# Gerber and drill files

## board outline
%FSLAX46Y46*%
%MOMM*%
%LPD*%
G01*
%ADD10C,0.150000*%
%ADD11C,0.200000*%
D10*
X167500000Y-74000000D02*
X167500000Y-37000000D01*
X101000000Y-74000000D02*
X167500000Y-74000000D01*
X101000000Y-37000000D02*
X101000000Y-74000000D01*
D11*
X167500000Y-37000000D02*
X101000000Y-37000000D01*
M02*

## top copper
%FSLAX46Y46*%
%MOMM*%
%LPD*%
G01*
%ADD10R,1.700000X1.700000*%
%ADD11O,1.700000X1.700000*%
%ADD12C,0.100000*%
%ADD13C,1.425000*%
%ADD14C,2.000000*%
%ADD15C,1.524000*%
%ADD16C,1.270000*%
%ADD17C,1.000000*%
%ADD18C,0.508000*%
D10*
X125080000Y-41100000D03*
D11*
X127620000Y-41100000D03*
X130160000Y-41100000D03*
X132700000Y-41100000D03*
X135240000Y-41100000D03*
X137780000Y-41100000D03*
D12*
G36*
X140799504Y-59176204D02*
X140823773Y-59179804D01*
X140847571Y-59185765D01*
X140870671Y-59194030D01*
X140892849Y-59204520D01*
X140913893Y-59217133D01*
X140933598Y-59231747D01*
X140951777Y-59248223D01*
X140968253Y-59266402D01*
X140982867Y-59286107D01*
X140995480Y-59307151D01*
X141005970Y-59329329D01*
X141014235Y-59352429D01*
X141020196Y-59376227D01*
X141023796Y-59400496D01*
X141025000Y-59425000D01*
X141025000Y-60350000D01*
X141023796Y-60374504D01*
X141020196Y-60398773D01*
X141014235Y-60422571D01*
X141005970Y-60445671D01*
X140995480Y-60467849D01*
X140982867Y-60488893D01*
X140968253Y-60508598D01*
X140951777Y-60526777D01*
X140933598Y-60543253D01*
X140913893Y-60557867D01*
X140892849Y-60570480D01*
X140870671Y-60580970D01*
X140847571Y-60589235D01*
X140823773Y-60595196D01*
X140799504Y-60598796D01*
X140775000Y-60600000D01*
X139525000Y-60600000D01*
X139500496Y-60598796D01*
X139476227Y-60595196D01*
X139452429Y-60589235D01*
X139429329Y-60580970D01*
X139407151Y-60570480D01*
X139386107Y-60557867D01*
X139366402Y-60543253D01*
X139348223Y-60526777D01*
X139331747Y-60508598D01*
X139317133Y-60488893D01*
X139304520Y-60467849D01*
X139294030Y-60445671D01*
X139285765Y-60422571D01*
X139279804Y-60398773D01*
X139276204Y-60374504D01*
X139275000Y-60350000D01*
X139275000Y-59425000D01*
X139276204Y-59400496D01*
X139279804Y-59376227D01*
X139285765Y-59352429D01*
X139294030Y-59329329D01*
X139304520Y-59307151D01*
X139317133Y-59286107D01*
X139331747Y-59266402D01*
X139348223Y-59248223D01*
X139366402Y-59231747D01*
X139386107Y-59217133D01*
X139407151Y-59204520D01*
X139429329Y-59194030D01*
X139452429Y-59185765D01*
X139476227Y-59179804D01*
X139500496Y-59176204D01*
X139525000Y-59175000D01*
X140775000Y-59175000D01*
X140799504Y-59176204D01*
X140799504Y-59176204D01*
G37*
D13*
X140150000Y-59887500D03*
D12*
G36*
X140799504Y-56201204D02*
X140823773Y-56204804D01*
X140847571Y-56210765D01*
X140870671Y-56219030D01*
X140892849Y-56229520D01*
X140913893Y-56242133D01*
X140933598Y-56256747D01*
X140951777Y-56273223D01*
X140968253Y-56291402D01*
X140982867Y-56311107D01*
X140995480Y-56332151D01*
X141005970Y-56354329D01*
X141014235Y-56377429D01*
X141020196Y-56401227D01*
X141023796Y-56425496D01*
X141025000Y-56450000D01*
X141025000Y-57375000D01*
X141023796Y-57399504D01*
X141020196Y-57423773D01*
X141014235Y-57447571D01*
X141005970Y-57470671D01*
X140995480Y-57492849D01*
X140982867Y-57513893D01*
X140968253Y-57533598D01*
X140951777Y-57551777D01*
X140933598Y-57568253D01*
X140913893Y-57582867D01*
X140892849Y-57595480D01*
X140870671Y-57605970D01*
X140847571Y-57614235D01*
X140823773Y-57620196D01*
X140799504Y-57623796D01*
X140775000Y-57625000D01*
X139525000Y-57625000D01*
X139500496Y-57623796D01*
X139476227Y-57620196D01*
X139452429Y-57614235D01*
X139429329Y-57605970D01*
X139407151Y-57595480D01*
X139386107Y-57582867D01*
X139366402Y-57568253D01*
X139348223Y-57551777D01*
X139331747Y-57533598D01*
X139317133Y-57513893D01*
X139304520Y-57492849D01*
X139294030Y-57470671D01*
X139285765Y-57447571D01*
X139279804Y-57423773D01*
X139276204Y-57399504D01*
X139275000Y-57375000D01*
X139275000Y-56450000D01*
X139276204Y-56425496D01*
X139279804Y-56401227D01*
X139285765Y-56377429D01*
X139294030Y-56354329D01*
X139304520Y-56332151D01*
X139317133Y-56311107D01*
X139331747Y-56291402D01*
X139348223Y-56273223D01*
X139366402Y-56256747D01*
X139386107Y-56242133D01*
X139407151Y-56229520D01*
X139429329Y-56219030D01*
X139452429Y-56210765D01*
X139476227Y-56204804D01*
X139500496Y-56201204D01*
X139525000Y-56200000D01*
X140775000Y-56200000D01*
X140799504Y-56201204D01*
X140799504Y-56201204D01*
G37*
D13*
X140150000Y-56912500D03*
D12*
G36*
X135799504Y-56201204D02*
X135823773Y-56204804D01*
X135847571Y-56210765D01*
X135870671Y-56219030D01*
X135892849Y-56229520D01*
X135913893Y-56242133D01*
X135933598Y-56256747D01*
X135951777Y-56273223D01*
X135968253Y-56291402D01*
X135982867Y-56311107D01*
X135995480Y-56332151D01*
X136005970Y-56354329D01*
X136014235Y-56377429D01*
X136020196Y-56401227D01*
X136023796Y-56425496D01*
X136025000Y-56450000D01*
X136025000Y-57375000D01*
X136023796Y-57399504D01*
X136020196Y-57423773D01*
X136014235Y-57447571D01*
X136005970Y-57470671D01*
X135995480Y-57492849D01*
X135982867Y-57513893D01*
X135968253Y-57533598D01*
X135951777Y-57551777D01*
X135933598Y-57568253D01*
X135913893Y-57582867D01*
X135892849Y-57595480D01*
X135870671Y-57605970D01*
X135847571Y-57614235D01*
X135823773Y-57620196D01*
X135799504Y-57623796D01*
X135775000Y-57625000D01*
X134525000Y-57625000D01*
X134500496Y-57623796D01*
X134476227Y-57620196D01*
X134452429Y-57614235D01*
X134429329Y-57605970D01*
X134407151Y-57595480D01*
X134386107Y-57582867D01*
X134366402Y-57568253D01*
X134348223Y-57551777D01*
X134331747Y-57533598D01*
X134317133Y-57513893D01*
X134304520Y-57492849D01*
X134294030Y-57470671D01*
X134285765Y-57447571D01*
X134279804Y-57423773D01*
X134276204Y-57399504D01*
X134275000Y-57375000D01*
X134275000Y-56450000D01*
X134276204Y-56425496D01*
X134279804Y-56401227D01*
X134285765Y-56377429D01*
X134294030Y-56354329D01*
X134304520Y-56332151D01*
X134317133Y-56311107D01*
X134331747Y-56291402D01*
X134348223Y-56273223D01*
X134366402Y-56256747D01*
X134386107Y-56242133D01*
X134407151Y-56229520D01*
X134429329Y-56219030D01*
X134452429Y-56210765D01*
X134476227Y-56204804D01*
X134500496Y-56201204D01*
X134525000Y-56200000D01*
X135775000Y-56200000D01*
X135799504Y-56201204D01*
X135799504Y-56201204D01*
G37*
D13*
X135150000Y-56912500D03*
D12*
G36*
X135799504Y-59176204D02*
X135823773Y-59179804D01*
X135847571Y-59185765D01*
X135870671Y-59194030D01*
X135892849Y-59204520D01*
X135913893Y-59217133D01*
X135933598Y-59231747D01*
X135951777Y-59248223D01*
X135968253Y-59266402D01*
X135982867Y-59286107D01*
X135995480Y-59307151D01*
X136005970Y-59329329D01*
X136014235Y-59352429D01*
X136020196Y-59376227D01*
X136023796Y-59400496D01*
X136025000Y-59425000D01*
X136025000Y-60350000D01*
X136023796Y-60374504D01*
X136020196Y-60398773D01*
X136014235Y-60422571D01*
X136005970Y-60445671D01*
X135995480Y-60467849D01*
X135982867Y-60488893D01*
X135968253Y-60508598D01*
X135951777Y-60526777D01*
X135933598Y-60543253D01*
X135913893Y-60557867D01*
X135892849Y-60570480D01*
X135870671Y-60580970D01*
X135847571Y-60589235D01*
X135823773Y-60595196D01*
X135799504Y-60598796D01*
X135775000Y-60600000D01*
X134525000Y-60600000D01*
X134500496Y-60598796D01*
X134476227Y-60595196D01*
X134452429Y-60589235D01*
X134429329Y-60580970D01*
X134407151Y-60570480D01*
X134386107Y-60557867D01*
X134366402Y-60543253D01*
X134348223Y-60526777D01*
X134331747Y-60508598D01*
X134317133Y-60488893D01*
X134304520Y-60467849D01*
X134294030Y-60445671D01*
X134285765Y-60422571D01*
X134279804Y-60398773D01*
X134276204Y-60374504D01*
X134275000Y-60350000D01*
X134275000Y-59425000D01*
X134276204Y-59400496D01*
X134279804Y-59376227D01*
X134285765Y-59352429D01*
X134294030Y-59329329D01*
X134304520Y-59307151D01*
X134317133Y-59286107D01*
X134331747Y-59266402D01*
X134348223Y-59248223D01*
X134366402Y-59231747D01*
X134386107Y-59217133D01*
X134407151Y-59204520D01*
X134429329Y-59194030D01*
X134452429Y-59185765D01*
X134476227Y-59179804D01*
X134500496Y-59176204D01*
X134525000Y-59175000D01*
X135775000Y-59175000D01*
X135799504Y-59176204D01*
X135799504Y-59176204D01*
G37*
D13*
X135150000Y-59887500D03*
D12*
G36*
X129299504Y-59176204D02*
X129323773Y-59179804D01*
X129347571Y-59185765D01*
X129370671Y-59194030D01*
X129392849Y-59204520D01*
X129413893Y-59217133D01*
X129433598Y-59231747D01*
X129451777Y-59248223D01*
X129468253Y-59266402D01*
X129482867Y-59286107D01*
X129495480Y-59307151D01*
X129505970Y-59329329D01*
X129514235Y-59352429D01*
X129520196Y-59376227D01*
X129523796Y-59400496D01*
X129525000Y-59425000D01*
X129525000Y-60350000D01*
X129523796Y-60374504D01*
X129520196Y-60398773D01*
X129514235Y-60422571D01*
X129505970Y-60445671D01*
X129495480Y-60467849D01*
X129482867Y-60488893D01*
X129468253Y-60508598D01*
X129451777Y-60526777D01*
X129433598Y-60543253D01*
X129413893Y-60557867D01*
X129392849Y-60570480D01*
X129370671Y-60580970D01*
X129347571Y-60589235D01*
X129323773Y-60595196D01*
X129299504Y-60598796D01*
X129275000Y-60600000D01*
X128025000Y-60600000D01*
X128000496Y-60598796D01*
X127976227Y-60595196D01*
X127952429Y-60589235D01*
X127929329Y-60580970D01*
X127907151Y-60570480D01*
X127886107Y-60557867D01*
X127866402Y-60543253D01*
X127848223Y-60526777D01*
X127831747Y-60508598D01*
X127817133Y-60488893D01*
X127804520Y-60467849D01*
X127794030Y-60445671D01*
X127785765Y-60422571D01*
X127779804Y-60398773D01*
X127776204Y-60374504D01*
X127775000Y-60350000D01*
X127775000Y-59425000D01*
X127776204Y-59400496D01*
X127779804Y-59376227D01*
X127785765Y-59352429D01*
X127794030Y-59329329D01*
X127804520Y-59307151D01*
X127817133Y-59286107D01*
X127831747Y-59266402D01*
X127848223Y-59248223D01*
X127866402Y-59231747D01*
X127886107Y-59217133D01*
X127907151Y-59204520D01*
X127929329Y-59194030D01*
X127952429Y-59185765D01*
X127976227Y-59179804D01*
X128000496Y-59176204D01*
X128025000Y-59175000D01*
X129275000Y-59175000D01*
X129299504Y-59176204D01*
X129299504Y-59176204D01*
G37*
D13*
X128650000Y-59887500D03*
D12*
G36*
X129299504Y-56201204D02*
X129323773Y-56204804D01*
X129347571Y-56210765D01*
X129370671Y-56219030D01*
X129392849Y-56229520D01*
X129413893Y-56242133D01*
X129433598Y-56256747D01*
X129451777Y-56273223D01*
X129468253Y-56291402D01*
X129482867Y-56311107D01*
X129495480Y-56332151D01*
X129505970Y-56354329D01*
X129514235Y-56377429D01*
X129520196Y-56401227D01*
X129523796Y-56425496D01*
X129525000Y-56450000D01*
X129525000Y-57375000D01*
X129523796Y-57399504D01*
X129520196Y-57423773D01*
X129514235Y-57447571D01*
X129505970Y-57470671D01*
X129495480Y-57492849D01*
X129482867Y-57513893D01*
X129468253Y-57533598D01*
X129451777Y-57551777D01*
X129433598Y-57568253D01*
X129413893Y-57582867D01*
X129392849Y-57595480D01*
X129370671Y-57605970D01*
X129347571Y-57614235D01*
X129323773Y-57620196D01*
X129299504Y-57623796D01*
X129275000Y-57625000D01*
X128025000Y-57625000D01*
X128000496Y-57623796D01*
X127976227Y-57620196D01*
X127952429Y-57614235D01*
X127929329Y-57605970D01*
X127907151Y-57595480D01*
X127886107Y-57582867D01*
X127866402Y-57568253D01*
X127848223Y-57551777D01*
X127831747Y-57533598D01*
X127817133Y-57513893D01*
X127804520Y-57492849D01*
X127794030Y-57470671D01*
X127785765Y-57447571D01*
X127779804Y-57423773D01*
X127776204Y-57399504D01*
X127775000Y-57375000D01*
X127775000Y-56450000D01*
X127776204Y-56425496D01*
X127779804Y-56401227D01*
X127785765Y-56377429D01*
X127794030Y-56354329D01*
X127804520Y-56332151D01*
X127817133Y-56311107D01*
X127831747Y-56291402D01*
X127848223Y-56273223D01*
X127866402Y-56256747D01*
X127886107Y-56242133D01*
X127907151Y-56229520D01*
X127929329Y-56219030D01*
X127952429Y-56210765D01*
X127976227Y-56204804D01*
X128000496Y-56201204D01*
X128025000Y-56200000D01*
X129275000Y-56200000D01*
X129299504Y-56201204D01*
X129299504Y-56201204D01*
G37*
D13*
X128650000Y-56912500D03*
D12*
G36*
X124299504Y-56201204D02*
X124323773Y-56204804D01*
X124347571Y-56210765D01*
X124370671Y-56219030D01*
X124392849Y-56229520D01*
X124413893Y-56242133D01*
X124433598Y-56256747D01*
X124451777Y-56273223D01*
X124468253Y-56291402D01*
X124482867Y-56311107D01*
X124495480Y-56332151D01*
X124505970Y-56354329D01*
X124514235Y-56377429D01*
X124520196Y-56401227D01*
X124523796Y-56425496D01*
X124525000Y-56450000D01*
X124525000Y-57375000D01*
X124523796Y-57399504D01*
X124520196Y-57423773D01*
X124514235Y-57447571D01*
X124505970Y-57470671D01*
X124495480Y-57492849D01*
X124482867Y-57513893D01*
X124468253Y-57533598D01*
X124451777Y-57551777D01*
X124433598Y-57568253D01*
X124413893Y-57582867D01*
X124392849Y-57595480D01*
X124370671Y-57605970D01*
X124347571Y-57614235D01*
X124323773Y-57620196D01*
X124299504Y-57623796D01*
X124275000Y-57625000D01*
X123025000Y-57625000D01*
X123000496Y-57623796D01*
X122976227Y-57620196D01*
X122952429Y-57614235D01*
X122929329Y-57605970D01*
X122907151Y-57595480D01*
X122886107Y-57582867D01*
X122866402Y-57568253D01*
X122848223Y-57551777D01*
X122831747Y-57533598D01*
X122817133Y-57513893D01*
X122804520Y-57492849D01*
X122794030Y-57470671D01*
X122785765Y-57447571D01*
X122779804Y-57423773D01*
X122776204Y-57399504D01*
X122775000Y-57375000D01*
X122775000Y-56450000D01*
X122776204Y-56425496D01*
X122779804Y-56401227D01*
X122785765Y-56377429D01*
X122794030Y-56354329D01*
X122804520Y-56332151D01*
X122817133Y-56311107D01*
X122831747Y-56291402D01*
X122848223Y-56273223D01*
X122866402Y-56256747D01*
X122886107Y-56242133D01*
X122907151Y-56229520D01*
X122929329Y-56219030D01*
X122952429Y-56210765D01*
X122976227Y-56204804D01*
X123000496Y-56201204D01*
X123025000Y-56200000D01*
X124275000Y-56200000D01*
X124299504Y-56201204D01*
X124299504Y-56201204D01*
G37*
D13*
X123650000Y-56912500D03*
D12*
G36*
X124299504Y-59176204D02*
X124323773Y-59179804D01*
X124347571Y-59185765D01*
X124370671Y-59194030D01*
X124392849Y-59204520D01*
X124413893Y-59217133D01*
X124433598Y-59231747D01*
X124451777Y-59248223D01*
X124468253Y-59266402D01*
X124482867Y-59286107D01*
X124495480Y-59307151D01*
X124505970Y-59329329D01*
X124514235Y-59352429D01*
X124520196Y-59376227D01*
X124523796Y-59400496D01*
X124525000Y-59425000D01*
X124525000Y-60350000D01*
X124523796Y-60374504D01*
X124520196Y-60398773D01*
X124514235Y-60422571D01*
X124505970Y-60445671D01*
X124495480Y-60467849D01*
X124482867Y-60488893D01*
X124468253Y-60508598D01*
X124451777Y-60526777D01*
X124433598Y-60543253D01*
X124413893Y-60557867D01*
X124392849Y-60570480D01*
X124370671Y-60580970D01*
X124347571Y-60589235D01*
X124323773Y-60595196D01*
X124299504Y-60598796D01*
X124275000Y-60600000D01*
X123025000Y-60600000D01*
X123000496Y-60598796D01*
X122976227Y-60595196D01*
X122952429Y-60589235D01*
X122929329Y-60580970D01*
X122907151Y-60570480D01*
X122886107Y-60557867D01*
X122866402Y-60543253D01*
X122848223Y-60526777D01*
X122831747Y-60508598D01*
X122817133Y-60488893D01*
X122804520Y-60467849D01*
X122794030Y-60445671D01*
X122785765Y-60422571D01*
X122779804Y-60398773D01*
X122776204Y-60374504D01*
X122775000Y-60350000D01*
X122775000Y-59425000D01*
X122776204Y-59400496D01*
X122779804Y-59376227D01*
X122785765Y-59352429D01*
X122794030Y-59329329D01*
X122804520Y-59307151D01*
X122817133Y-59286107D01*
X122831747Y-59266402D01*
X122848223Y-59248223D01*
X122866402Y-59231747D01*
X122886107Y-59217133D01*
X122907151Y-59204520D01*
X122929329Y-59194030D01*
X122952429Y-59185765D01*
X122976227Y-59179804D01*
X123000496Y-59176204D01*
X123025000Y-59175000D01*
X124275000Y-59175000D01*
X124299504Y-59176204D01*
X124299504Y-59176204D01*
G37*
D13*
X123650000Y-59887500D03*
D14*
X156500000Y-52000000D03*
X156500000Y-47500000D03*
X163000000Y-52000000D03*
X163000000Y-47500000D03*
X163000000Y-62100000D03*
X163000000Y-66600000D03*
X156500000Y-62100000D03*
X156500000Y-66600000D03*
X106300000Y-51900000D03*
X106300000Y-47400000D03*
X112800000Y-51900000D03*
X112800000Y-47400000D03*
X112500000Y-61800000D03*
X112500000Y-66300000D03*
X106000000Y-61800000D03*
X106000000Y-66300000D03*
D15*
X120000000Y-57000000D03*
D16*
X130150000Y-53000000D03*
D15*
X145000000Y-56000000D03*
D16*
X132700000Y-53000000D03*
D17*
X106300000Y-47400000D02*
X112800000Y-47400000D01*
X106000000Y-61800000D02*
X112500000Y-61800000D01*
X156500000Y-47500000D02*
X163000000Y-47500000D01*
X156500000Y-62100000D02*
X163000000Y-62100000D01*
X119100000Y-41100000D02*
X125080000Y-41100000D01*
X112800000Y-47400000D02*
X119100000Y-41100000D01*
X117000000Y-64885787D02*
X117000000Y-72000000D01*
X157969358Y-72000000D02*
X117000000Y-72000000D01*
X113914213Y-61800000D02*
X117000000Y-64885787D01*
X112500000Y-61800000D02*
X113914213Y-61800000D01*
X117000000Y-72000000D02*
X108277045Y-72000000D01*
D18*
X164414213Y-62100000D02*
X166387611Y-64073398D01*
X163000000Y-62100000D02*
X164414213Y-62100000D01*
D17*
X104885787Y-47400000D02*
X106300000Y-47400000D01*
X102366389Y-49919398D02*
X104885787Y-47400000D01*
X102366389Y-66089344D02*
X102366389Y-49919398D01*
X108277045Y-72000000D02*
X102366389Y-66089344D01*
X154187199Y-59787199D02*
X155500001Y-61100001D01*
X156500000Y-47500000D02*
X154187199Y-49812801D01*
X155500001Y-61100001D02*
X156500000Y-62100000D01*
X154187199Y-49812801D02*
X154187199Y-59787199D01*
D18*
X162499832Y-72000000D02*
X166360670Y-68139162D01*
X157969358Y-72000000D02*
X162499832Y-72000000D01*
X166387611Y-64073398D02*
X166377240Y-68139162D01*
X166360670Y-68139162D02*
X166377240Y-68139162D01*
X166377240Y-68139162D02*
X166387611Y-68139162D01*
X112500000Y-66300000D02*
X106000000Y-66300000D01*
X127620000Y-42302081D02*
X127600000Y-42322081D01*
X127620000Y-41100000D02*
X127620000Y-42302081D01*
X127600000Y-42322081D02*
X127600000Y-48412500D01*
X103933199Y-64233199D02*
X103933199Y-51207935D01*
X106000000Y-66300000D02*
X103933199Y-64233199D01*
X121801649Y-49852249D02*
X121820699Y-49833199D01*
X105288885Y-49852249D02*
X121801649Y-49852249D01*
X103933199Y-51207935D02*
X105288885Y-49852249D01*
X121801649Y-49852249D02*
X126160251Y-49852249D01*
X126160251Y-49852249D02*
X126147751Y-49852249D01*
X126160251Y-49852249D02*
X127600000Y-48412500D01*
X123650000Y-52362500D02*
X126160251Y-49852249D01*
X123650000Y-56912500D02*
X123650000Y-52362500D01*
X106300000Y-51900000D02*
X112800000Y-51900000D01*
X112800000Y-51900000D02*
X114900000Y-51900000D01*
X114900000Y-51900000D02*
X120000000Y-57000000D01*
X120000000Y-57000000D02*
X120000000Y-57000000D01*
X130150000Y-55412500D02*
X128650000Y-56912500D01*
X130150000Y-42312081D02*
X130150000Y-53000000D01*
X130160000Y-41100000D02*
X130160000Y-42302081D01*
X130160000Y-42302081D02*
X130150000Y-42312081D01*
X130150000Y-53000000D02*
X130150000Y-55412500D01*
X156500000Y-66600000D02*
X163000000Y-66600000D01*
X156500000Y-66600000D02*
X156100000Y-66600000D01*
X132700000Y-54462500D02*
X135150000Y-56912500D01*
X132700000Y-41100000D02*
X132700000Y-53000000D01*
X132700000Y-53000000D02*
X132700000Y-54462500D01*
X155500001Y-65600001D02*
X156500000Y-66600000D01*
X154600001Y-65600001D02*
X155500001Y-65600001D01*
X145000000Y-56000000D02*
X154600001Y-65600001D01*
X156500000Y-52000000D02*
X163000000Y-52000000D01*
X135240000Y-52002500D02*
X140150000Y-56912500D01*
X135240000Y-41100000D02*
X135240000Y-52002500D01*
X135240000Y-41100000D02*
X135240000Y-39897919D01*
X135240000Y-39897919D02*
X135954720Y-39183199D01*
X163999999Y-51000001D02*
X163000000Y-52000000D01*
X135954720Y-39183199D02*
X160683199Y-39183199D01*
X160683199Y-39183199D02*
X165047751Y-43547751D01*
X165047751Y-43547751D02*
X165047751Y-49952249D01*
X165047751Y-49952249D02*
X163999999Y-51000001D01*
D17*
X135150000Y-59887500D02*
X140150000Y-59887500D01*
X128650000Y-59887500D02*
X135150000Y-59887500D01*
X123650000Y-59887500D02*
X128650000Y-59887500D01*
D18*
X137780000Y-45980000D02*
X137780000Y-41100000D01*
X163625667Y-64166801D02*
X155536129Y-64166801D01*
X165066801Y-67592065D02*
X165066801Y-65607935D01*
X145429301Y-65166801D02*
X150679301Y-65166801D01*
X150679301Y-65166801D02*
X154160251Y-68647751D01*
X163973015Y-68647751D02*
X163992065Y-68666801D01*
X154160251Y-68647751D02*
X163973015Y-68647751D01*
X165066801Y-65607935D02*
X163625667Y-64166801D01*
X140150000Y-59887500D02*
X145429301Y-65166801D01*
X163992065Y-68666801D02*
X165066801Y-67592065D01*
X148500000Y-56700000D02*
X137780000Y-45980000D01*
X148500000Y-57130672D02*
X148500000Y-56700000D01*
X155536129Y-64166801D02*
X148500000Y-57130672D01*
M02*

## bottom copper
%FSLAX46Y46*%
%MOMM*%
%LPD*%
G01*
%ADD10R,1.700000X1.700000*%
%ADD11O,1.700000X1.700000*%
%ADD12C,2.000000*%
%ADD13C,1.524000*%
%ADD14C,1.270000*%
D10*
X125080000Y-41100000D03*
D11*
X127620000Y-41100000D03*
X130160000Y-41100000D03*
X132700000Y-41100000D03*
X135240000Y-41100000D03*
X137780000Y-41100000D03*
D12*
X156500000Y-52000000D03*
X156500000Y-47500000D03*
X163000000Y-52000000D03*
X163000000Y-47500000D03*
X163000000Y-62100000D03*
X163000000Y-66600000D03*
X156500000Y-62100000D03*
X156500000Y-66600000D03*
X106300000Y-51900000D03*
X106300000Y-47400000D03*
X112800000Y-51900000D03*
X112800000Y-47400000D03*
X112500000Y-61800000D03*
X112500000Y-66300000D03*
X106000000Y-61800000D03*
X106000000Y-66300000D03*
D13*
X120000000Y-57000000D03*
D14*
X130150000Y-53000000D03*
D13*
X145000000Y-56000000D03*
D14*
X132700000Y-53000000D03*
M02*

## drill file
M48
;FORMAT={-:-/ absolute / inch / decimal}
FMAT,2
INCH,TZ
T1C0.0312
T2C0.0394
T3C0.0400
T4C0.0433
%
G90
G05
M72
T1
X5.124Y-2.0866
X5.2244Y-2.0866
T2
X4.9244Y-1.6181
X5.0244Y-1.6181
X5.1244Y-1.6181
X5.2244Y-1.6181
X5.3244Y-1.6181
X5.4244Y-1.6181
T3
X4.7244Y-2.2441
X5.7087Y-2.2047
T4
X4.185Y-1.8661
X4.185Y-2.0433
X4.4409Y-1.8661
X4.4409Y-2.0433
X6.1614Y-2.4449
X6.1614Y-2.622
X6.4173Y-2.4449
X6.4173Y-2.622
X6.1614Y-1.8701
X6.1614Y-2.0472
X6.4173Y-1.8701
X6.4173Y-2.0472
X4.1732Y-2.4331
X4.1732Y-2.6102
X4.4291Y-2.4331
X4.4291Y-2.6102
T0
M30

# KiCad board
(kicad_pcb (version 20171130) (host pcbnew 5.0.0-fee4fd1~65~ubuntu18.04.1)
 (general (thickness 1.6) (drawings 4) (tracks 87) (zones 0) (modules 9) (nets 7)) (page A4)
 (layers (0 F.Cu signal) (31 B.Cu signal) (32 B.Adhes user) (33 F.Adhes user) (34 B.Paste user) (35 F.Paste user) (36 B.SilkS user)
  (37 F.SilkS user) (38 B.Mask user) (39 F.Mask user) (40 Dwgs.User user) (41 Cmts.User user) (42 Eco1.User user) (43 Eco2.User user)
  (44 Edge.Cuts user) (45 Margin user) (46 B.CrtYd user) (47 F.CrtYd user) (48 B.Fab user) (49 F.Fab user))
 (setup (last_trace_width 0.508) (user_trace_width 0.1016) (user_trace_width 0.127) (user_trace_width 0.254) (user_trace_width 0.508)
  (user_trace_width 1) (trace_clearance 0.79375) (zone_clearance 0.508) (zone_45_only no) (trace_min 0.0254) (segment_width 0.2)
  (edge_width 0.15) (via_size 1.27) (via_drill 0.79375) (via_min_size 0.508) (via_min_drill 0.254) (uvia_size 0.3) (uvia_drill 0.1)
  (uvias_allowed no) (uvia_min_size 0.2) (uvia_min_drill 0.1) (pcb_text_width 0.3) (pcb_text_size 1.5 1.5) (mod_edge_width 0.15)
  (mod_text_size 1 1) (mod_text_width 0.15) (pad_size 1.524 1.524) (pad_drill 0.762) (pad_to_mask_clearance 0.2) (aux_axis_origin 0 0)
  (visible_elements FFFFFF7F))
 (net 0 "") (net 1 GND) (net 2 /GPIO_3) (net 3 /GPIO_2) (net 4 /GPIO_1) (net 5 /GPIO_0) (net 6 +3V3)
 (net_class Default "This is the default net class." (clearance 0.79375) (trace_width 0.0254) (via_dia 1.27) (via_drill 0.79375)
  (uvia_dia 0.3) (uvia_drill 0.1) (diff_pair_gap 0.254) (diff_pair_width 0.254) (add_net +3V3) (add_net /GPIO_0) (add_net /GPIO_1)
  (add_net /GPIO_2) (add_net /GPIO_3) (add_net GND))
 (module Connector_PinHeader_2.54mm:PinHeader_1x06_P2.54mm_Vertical (layer F.Cu) (at 125.08 41.1 90)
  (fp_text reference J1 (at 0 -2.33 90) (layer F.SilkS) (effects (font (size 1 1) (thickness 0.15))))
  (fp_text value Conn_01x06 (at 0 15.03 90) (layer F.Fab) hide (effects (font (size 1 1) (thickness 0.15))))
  (pad 1 thru_hole rect (at 0 0 90) (size 1.7 1.7) (drill 1) (layers *.Cu *.Mask) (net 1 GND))
  (pad 2 thru_hole oval (at 0 2.54 90) (size 1.7 1.7) (drill 1) (layers *.Cu *.Mask) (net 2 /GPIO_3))
  (pad 3 thru_hole oval (at 0 5.08 90) (size 1.7 1.7) (drill 1) (layers *.Cu *.Mask) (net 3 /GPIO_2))
  (pad 4 thru_hole oval (at 0 7.62 90) (size 1.7 1.7) (drill 1) (layers *.Cu *.Mask) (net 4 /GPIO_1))
  (pad 5 thru_hole oval (at 0 10.16 90) (size 1.7 1.7) (drill 1) (layers *.Cu *.Mask) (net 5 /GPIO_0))
  (pad 6 thru_hole oval (at 0 12.7 90) (size 1.7 1.7) (drill 1) (layers *.Cu *.Mask) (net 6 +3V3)))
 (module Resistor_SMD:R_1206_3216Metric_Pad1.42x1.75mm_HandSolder (layer F.Cu) (at 140.15 58.4 90)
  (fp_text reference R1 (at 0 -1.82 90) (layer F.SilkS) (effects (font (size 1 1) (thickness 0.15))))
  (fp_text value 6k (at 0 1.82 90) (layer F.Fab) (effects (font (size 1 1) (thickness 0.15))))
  (pad 1 smd roundrect (at -1.4875 0 90) (size 1.425 1.75) (layers F.Cu F.Paste F.Mask) (roundrect_rratio 0.175439) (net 6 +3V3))
  (pad 2 smd roundrect (at 1.4875 0 90) (size 1.425 1.75) (layers F.Cu F.Paste F.Mask) (roundrect_rratio 0.175439) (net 5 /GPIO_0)))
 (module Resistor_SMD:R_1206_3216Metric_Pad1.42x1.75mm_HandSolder (layer F.Cu) (at 135.15 58.4 90)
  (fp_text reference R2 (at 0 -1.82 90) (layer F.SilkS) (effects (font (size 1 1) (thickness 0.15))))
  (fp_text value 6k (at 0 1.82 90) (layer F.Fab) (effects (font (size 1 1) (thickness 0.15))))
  (pad 2 smd roundrect (at 1.4875 0 90) (size 1.425 1.75) (layers F.Cu F.Paste F.Mask) (roundrect_rratio 0.175439) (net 4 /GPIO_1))
  (pad 1 smd roundrect (at -1.4875 0 90) (size 1.425 1.75) (layers F.Cu F.Paste F.Mask) (roundrect_rratio 0.175439) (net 6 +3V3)))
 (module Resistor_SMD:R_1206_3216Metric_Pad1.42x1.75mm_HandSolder (layer F.Cu) (at 128.65 58.4 90)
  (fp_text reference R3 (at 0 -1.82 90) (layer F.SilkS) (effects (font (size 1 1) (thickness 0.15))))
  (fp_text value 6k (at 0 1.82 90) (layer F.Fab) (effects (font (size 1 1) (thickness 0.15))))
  (pad 1 smd roundrect (at -1.4875 0 90) (size 1.425 1.75) (layers F.Cu F.Paste F.Mask) (roundrect_rratio 0.175439) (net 6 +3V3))
  (pad 2 smd roundrect (at 1.4875 0 90) (size 1.425 1.75) (layers F.Cu F.Paste F.Mask) (roundrect_rratio 0.175439) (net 3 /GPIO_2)))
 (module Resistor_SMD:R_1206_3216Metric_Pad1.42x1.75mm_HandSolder (layer F.Cu) (at 123.65 58.4 90)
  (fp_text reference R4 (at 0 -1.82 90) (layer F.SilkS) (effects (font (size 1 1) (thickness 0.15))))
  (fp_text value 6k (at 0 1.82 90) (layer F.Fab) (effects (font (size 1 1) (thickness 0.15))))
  (pad 2 smd roundrect (at 1.4875 0 90) (size 1.425 1.75) (layers F.Cu F.Paste F.Mask) (roundrect_rratio 0.175439) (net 2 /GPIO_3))
  (pad 1 smd roundrect (at -1.4875 0 90) (size 1.425 1.75) (layers F.Cu F.Paste F.Mask) (roundrect_rratio 0.175439) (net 6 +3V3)))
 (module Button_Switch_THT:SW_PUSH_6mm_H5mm (layer F.Cu) (at 156.5 47.5)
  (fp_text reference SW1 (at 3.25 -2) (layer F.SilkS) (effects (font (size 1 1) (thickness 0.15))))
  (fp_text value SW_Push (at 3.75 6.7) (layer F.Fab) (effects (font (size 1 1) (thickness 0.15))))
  (pad 2 thru_hole circle (at 0 4.5 90) (size 2 2) (drill 1.1) (layers *.Cu *.Mask) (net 5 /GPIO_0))
  (pad 1 thru_hole circle (at 0 0 90) (size 2 2) (drill 1.1) (layers *.Cu *.Mask) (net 1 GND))
  (pad 2 thru_hole circle (at 6.5 4.5 90) (size 2 2) (drill 1.1) (layers *.Cu *.Mask) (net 5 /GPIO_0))
  (pad 1 thru_hole circle (at 6.5 0 90) (size 2 2) (drill 1.1) (layers *.Cu *.Mask) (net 1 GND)))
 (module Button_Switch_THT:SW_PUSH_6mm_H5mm (layer F.Cu) (at 156.5 62.1)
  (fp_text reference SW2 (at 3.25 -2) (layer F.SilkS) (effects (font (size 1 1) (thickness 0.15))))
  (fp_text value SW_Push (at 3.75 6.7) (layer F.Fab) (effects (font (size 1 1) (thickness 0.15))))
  (pad 1 thru_hole circle (at 6.5 0 90) (size 2 2) (drill 1.1) (layers *.Cu *.Mask) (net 1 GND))
  (pad 2 thru_hole circle (at 6.5 4.5 90) (size 2 2) (drill 1.1) (layers *.Cu *.Mask) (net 4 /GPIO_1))
  (pad 1 thru_hole circle (at 0 0 90) (size 2 2) (drill 1.1) (layers *.Cu *.Mask) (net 1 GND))
  (pad 2 thru_hole circle (at 0 4.5 90) (size 2 2) (drill 1.1) (layers *.Cu *.Mask) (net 4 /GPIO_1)))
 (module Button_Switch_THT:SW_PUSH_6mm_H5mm (layer F.Cu) (at 106.3 47.4)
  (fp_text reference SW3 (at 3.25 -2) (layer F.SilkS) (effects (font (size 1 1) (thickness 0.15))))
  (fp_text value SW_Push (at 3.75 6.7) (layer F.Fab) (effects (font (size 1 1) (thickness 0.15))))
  (pad 2 thru_hole circle (at 0 4.5 90) (size 2 2) (drill 1.1) (layers *.Cu *.Mask) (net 3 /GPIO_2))
  (pad 1 thru_hole circle (at 0 0 90) (size 2 2) (drill 1.1) (layers *.Cu *.Mask) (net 1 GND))
  (pad 2 thru_hole circle (at 6.5 4.5 90) (size 2 2) (drill 1.1) (layers *.Cu *.Mask) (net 3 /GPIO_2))
  (pad 1 thru_hole circle (at 6.5 0 90) (size 2 2) (drill 1.1) (layers *.Cu *.Mask) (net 1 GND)))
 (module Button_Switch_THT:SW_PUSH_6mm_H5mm (layer F.Cu) (at 106 61.8)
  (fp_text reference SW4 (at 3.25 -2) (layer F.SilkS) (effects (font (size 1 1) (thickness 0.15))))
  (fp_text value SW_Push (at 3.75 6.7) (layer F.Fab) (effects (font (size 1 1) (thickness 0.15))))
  (pad 1 thru_hole circle (at 6.5 0 90) (size 2 2) (drill 1.1) (layers *.Cu *.Mask) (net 1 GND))
  (pad 2 thru_hole circle (at 6.5 4.5 90) (size 2 2) (drill 1.1) (layers *.Cu *.Mask) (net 2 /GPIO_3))
  (pad 1 thru_hole circle (at 0 0 90) (size 2 2) (drill 1.1) (layers *.Cu *.Mask) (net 1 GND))
  (pad 2 thru_hole circle (at 0 4.5 90) (size 2 2) (drill 1.1) (layers *.Cu *.Mask) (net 2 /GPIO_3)))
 (gr_line (start 167.5 74) (end 167.5 37) (layer Edge.Cuts) (width 0.15))
 (gr_line (start 101 74) (end 167.5 74) (layer Edge.Cuts) (width 0.15))
 (gr_line (start 101 37) (end 101 74) (layer Edge.Cuts) (width 0.15))
 (gr_line (start 167.5 37) (end 101 37) (layer Edge.Cuts) (width 0.2))
 (segment (start 106.3 47.4) (end 112.8 47.4) (width 1) (layer F.Cu) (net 1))
 (segment (start 106 61.8) (end 112.5 61.8) (width 1) (layer F.Cu) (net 1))
 (segment (start 156.5 47.5) (end 163 47.5) (width 1) (layer F.Cu) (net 1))
 (segment (start 156.5 62.1) (end 163 62.1) (width 1) (layer F.Cu) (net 1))
 (segment (start 119.1 41.1) (end 125.08 41.1) (width 1) (layer F.Cu) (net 1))
 (segment (start 112.8 47.4) (end 119.1 41.1) (width 1) (layer F.Cu) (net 1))
 (segment (start 117 64.885787) (end 117 72) (width 1) (layer F.Cu) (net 1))
 (segment (start 157.969358 72) (end 117 72) (width 1) (layer F.Cu) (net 1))
 (segment (start 113.914213 61.8) (end 117 64.885787) (width 1) (layer F.Cu) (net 1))
 (segment (start 112.5 61.8) (end 113.914213 61.8) (width 1) (layer F.Cu) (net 1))
 (segment (start 117 72) (end 108.277045 72) (width 1) (layer F.Cu) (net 1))
 (segment (start 164.414213 62.1) (end 166.387611 64.073398) (width 0.508) (layer F.Cu) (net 1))
 (segment (start 163 62.1) (end 164.414213 62.1) (width 0.508) (layer F.Cu) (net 1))
 (segment (start 104.885787 47.4) (end 106.3 47.4) (width 1) (layer F.Cu) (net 1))
 (segment (start 102.366389 49.919398) (end 104.885787 47.4) (width 1) (layer F.Cu) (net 1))
 (segment (start 102.366389 66.089344) (end 102.366389 49.919398) (width 1) (layer F.Cu) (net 1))
 (segment (start 108.277045 72) (end 102.366389 66.089344) (width 1) (layer F.Cu) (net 1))
 (segment (start 154.187199 59.787199) (end 155.500001 61.100001) (width 1) (layer F.Cu) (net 1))
 (segment (start 156.5 47.5) (end 154.187199 49.812801) (width 1) (layer F.Cu) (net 1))
 (segment (start 155.500001 61.100001) (end 156.5 62.1) (width 1) (layer F.Cu) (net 1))
 (segment (start 154.187199 49.812801) (end 154.187199 59.787199) (width 1) (layer F.Cu) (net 1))
 (segment (start 162.499832 72) (end 166.36067 68.139162) (width 0.508) (layer F.Cu) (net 1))
 (segment (start 157.969358 72) (end 162.499832 72) (width 0.508) (layer F.Cu) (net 1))
 (segment (start 166.387611 64.073398) (end 166.37724 68.139162) (width 0.508) (layer F.Cu) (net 1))
 (segment (start 166.36067 68.139162) (end 166.37724 68.139162) (width 0.508) (layer F.Cu) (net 1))
 (segment (start 166.37724 68.139162) (end 166.387611 68.139162) (width 0.508) (layer F.Cu) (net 1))
 (segment (start 112.5 66.3) (end 106 66.3) (width 0.508) (layer F.Cu) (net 2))
 (segment (start 127.62 42.302081) (end 127.6 42.322081) (width 0.508) (layer F.Cu) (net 2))
 (segment (start 127.62 41.1) (end 127.62 42.302081) (width 0.508) (layer F.Cu) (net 2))
 (segment (start 127.6 42.322081) (end 127.6 48.4125) (width 0.508) (layer F.Cu) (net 2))
 (segment (start 103.933199 64.233199) (end 103.933199 51.207935) (width 0.508) (layer F.Cu) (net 2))
 (segment (start 106 66.3) (end 103.933199 64.233199) (width 0.508) (layer F.Cu) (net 2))
 (segment (start 121.801649 49.852249) (end 121.820699 49.833199) (width 0.508) (layer F.Cu) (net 2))
 (segment (start 105.288885 49.852249) (end 121.801649 49.852249) (width 0.508) (layer F.Cu) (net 2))
 (segment (start 103.933199 51.207935) (end 105.288885 49.852249) (width 0.508) (layer F.Cu) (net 2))
 (segment (start 121.801649 49.852249) (end 126.160251 49.852249) (width 0.508) (layer F.Cu) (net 2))
 (segment (start 126.160251 49.852249) (end 126.147751 49.852249) (width 0.508) (layer F.Cu) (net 2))
 (segment (start 126.160251 49.852249) (end 127.6 48.4125) (width 0.508) (layer F.Cu) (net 2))
 (segment (start 123.65 52.3625) (end 126.160251 49.852249) (width 0.508) (layer F.Cu) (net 2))
 (segment (start 123.65 56.9125) (end 123.65 52.3625) (width 0.508) (layer F.Cu) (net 2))
 (segment (start 106.3 51.9) (end 112.8 51.9) (width 0.508) (layer F.Cu) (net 3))
 (segment (start 112.8 51.9) (end 114.9 51.9) (width 0.508) (layer F.Cu) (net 3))
 (segment (start 114.9 51.9) (end 120 57) (width 0.508) (layer F.Cu) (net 3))
 (segment (start 120 57) (end 120 57) (width 0.508) (layer F.Cu) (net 3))
 (via (at 120 57) (size 1.524) (drill 1.016) (layers F.Cu B.Cu) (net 3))
 (segment (start 130.15 55.4125) (end 128.65 56.9125) (width 0.508) (layer F.Cu) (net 3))
 (segment (start 130.15 42.312081) (end 130.15 53) (width 0.508) (layer F.Cu) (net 3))
 (segment (start 130.16 41.1) (end 130.16 42.302081) (width 0.508) (layer F.Cu) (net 3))
 (segment (start 130.16 42.302081) (end 130.15 42.312081) (width 0.508) (layer F.Cu) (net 3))
 (segment (start 130.15 53) (end 130.15 55.4125) (width 0.508) (layer F.Cu) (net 3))
 (via (at 130.15 53) (size 1.27) (drill 0.79375) (layers F.Cu B.Cu) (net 3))
 (segment (start 156.5 66.6) (end 163 66.6) (width 0.508) (layer F.Cu) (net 4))
 (segment (start 156.5 66.6) (end 156.1 66.6) (width 0.508) (layer F.Cu) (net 4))
 (via (at 145 56) (size 1.524) (drill 1.016) (layers F.Cu B.Cu) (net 4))
 (segment (start 132.7 54.4625) (end 135.15 56.9125) (width 0.508) (layer F.Cu) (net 4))
 (segment (start 132.7 41.1) (end 132.7 53) (width 0.508) (layer F.Cu) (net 4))
 (segment (start 132.7 53) (end 132.7 54.4625) (width 0.508) (layer F.Cu) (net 4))
 (via (at 132.7 53) (size 1.27) (drill 0.79375) (layers F.Cu B.Cu) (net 4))
 (segment (start 155.500001 65.600001) (end 156.5 66.6) (width 0.508) (layer F.Cu) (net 4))
 (segment (start 154.600001 65.600001) (end 155.500001 65.600001) (width 0.508) (layer F.Cu) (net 4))
 (segment (start 145 56) (end 154.600001 65.600001) (width 0.508) (layer F.Cu) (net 4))
 (segment (start 156.5 52) (end 163 52) (width 0.508) (layer F.Cu) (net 5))
 (segment (start 135.24 52.0025) (end 140.15 56.9125) (width 0.508) (layer F.Cu) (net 5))
 (segment (start 135.24 41.1) (end 135.24 52.0025) (width 0.508) (layer F.Cu) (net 5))
 (segment (start 135.24 41.1) (end 135.24 39.897919) (width 0.508) (layer F.Cu) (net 5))
 (segment (start 135.24 39.897919) (end 135.95472 39.183199) (width 0.508) (layer F.Cu) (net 5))
 (segment (start 163.999999 51.000001) (end 163 52) (width 0.508) (layer F.Cu) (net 5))
 (segment (start 135.95472 39.183199) (end 160.683199 39.183199) (width 0.508) (layer F.Cu) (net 5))
 (segment (start 160.683199 39.183199) (end 165.047751 43.547751) (width 0.508) (layer F.Cu) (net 5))
 (segment (start 165.047751 43.547751) (end 165.047751 49.952249) (width 0.508) (layer F.Cu) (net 5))
 (segment (start 165.047751 49.952249) (end 163.999999 51.000001) (width 0.508) (layer F.Cu) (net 5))
 (segment (start 135.15 59.8875) (end 140.15 59.8875) (width 1) (layer F.Cu) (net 6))
 (segment (start 128.65 59.8875) (end 135.15 59.8875) (width 1) (layer F.Cu) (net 6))
 (segment (start 123.65 59.8875) (end 128.65 59.8875) (width 1) (layer F.Cu) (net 6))
 (segment (start 137.78 45.98) (end 137.78 41.1) (width 0.508) (layer F.Cu) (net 6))
 (segment (start 163.625667 64.166801) (end 155.536129 64.166801) (width 0.508) (layer F.Cu) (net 6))
 (segment (start 165.066801 67.592065) (end 165.066801 65.607935) (width 0.508) (layer F.Cu) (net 6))
 (segment (start 145.429301 65.166801) (end 150.679301 65.166801) (width 0.508) (layer F.Cu) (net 6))
 (segment (start 150.679301 65.166801) (end 154.160251 68.647751) (width 0.508) (layer F.Cu) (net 6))
 (segment (start 163.973015 68.647751) (end 163.992065 68.666801) (width 0.508) (layer F.Cu) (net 6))
 (segment (start 154.160251 68.647751) (end 163.973015 68.647751) (width 0.508) (layer F.Cu) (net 6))
 (segment (start 165.066801 65.607935) (end 163.625667 64.166801) (width 0.508) (layer F.Cu) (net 6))
 (segment (start 140.15 59.8875) (end 145.429301 65.166801) (width 0.508) (layer F.Cu) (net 6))
 (segment (start 163.992065 68.666801) (end 165.066801 67.592065) (width 0.508) (layer F.Cu) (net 6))
 (segment (start 148.5 56.7) (end 137.78 45.98) (width 0.508) (layer F.Cu) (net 6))
 (segment (start 148.5 57.130672) (end 148.5 56.7) (width 0.508) (layer F.Cu) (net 6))
 (segment (start 155.536129 64.166801) (end 148.5 57.130672) (width 0.508) (layer F.Cu) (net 6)))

